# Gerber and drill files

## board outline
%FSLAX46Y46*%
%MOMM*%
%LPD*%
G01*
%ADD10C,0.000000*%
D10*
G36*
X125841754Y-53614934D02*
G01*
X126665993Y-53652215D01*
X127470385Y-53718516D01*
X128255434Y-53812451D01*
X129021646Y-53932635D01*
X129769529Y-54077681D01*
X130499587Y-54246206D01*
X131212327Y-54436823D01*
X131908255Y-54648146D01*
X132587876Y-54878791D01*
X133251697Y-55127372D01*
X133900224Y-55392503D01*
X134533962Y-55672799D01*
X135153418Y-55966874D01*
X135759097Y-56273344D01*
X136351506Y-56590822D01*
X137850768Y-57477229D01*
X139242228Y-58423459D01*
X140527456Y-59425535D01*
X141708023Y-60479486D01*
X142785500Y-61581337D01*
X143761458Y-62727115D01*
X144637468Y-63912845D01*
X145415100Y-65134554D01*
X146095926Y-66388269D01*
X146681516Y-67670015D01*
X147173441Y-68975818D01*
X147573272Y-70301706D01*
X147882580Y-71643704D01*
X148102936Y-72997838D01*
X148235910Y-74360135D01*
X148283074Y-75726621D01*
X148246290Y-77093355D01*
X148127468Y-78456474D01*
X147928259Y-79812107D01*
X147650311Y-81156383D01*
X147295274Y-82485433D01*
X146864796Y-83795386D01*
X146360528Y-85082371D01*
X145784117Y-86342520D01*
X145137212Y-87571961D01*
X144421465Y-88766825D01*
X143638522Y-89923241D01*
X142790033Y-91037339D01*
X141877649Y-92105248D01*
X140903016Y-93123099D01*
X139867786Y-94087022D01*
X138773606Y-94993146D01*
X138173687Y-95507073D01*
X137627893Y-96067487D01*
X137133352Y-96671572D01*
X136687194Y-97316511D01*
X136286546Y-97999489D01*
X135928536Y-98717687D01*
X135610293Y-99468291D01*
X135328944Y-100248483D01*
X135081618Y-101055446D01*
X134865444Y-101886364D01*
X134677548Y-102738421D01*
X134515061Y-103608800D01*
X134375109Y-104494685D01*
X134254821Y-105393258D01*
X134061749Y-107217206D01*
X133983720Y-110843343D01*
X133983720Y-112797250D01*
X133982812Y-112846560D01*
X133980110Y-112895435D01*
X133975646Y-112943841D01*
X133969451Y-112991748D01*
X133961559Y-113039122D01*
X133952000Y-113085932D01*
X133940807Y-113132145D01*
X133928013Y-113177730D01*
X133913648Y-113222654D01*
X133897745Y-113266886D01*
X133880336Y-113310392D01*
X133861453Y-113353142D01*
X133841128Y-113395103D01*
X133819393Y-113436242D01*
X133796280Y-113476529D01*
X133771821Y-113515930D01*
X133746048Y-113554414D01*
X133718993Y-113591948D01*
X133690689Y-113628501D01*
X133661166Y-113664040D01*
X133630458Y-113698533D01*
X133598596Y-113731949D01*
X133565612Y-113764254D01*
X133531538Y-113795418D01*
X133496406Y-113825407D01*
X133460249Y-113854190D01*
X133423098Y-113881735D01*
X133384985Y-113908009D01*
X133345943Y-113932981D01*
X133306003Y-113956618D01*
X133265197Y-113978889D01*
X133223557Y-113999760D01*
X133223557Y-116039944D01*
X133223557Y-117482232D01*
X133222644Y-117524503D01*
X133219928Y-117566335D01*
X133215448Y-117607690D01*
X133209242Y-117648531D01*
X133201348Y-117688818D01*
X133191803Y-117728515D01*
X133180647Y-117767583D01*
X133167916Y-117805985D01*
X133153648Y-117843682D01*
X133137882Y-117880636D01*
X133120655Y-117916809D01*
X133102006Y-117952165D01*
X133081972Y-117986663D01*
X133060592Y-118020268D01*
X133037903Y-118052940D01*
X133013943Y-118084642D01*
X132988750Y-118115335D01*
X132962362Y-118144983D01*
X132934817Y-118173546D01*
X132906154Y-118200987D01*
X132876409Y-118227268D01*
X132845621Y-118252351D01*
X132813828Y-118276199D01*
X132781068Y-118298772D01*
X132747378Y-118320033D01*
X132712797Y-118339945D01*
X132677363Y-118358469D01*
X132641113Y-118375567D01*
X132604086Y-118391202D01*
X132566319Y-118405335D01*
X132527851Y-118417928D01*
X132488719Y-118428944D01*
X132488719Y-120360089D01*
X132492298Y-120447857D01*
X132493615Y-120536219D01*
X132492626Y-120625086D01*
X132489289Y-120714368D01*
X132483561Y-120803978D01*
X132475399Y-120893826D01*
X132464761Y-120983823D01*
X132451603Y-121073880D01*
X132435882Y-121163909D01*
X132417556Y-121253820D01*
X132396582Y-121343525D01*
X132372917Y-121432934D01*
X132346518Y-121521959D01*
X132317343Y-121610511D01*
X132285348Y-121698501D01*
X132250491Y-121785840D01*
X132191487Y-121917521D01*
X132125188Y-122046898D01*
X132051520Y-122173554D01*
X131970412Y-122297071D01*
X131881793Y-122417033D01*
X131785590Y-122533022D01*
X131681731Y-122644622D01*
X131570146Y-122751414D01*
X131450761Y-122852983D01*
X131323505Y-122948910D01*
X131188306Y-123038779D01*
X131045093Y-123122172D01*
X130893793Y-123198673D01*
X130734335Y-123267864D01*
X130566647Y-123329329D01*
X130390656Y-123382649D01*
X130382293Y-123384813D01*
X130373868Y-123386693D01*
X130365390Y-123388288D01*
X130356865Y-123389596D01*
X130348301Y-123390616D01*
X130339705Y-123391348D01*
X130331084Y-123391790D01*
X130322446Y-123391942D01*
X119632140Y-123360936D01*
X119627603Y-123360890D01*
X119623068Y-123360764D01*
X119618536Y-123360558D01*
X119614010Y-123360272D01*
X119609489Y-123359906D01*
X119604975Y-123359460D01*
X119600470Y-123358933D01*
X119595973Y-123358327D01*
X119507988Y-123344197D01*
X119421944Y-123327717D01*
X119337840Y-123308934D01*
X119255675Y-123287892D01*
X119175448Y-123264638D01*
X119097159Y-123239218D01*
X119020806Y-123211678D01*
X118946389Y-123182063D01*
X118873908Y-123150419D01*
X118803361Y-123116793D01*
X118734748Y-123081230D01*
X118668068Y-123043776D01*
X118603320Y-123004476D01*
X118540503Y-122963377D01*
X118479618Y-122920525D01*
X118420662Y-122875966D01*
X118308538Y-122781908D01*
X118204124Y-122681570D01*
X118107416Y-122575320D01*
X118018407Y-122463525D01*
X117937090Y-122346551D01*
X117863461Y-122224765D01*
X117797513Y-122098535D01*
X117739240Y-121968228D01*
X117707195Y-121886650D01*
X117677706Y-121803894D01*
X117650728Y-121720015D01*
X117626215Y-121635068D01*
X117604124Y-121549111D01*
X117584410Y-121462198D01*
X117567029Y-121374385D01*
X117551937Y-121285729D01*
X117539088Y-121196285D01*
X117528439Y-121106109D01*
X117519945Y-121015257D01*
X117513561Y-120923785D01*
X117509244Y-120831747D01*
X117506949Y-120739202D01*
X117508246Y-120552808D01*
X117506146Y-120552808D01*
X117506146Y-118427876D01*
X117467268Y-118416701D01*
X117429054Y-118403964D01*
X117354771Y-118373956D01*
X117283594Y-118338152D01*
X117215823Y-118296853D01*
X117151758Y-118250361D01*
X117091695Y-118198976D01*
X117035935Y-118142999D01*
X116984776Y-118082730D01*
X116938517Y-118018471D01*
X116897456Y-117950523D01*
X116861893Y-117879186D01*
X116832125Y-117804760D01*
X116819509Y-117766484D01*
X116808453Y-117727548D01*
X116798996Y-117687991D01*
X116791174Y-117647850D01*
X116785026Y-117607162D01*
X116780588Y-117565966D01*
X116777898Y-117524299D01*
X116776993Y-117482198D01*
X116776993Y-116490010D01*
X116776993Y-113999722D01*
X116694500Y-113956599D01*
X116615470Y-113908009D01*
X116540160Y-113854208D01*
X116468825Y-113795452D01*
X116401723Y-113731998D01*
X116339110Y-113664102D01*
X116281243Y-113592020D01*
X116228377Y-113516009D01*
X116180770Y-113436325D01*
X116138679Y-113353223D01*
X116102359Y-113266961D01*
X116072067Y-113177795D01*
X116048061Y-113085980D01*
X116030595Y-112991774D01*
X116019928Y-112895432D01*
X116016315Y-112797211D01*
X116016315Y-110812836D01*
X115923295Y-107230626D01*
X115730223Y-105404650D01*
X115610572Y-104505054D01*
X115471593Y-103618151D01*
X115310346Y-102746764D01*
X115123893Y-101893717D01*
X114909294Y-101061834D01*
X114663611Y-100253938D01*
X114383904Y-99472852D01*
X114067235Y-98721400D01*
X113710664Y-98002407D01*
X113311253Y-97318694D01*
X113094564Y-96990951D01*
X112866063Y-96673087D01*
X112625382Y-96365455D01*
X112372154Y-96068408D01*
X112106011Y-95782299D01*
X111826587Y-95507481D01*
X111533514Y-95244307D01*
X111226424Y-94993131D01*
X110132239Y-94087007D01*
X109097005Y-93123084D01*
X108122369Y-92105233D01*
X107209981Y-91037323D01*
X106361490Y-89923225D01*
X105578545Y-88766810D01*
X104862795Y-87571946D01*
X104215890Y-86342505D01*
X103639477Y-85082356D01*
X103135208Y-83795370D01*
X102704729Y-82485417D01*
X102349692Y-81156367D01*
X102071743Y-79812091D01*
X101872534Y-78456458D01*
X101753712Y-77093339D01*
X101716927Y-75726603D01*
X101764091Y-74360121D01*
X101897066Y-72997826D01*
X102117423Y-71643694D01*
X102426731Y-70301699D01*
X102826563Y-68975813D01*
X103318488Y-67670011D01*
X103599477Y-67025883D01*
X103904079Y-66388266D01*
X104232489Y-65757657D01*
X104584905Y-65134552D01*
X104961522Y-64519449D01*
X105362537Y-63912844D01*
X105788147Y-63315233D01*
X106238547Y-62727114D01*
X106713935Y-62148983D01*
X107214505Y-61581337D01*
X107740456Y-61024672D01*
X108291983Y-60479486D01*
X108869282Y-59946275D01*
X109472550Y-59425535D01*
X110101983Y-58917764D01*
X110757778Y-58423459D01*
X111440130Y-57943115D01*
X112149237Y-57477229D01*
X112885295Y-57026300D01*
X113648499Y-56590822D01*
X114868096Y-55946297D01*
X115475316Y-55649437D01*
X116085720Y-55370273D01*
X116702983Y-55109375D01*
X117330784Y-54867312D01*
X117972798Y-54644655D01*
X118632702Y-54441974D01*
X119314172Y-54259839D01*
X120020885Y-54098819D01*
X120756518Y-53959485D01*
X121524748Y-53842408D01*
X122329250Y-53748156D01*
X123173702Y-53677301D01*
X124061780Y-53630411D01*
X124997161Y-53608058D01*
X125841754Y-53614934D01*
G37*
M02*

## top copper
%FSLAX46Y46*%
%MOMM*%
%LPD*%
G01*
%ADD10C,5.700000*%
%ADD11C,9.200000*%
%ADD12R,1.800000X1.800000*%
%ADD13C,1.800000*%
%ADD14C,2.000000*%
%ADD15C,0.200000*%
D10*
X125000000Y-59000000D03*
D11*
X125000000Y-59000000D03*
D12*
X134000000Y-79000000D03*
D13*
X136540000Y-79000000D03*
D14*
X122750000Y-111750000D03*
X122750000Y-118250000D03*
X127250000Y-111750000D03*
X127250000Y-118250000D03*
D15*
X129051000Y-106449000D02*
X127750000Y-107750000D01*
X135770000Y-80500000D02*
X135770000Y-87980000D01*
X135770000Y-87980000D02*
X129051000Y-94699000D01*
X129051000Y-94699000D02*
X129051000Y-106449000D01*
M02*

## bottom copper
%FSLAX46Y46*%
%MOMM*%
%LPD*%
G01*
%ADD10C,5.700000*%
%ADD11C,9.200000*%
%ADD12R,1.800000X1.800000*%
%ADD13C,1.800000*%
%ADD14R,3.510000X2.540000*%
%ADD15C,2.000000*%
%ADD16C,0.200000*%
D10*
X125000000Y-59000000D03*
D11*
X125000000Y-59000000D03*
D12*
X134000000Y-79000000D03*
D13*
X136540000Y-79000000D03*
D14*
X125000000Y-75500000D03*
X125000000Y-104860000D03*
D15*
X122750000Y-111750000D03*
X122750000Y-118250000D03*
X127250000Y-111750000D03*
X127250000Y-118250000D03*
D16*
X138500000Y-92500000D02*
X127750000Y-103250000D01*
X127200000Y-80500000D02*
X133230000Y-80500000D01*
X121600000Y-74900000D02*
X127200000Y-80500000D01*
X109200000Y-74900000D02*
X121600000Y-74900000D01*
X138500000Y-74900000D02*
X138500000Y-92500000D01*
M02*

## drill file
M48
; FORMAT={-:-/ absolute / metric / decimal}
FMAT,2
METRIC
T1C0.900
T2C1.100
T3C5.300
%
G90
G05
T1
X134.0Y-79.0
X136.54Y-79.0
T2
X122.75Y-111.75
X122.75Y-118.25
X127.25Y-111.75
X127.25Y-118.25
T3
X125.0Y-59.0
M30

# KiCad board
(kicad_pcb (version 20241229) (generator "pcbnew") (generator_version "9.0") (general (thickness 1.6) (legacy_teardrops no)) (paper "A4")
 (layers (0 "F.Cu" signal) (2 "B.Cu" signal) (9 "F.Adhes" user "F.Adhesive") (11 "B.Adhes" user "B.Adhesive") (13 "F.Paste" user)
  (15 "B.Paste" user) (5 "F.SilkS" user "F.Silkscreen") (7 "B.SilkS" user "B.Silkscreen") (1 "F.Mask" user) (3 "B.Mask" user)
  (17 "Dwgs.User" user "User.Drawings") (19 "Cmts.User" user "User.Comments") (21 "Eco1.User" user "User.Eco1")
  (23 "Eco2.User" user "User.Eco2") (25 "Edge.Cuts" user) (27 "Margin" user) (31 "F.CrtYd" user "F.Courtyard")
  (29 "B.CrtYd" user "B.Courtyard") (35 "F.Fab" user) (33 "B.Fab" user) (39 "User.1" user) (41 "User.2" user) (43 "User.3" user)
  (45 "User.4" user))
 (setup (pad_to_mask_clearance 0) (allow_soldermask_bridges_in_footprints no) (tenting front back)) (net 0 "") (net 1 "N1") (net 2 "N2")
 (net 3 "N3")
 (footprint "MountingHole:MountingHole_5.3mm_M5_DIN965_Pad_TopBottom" (layer "F.Cu") (at 125 59)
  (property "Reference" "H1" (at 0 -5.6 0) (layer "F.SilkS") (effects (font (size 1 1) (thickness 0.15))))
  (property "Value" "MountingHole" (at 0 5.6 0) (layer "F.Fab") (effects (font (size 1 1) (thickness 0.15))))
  (pad "1" thru_hole circle (at 0 0) (size 5.7 5.7) (drill 5.3) (layers "*.Cu" "*.Mask") (remove_unused_layers no))
  (pad "1" connect circle (at 0 0) (size 9.2 9.2) (layers "F.Cu" "F.Mask"))
  (pad "1" connect circle (at 0 0) (size 9.2 9.2) (layers "B.Cu" "B.Mask")))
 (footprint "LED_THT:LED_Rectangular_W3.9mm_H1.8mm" (layer "F.Cu") (at 134 79)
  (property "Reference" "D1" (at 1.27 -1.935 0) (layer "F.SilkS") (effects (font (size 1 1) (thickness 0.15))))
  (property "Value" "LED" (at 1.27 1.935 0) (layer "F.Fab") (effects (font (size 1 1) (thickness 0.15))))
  (pad "1" thru_hole rect (at 0 0) (size 1.8 1.8) (drill 0.9) (layers "*.Cu" "*.Mask") (remove_unused_layers no) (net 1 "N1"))
  (pad "2" thru_hole circle (at 2.54 0) (size 1.8 1.8) (drill 0.9) (layers "*.Cu" "*.Mask") (remove_unused_layers no) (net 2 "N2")))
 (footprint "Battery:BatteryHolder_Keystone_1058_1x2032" (layer "B.Cu") (at 125 90.18 -90)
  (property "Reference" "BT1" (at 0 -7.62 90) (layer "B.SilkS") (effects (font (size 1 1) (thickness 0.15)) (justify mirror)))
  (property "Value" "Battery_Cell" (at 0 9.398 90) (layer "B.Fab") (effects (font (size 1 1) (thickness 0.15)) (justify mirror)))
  (pad "1" smd rect (at -14.68 0 270) (size 2.54 3.51) (layers "B.Cu" "B.Mask" "B.Paste") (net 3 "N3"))
  (pad "2" smd rect (at 14.68 0 270) (size 2.54 3.51) (layers "B.Cu" "B.Mask" "B.Paste") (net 1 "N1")))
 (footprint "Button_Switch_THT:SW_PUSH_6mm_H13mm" (layer "B.Cu") (at 122.75 111.75 -90)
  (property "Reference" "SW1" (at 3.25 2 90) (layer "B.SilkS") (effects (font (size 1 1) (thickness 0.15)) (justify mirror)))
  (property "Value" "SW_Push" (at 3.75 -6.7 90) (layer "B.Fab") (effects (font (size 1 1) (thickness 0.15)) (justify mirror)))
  (pad "1" thru_hole circle (at 0 0 180) (size 2 2) (drill 1.1) (layers "*.Cu" "*.Mask") (remove_unused_layers no) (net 3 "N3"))
  (pad "1" thru_hole circle (at 6.5 0 180) (size 2 2) (drill 1.1) (layers "*.Cu" "*.Mask") (remove_unused_layers no) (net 3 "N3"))
  (pad "2" thru_hole circle (at 0 -4.5 180) (size 2 2) (drill 1.1) (layers "*.Cu" "*.Mask") (remove_unused_layers no) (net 2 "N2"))
  (pad "2" thru_hole circle (at 6.5 -4.5 180) (size 2 2) (drill 1.1) (layers "*.Cu" "*.Mask") (remove_unused_layers no) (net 2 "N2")))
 (gr_poly
  (pts (xy 125.841754 53.614934) (xy 126.665993 53.652215) (xy 127.470385 53.718516) (xy 128.255434 53.812451) (xy 129.021646 53.932635)
   (xy 129.769529 54.077681) (xy 130.499587 54.246206) (xy 131.212327 54.436823) (xy 131.908255 54.648146) (xy 132.587876 54.878791)
   (xy 133.251697 55.127372) (xy 133.900224 55.392503) (xy 134.533962 55.672799) (xy 135.153418 55.966874) (xy 135.759097 56.273344)
   (xy 136.351506 56.590822) (xy 137.850768 57.477229) (xy 139.242228 58.423459) (xy 140.527456 59.425535) (xy 141.708023 60.479486)
   (xy 142.7855 61.581337) (xy 143.761458 62.727115) (xy 144.637468 63.912845) (xy 145.4151 65.134554) (xy 146.095926 66.388269)
   (xy 146.681516 67.670015) (xy 147.173441 68.975818) (xy 147.573272 70.301706) (xy 147.88258 71.643704) (xy 148.102936 72.997838)
   (xy 148.23591 74.360135) (xy 148.283074 75.726621) (xy 148.24629 77.093355) (xy 148.127468 78.456474) (xy 147.928259 79.812107)
   (xy 147.650311 81.156383) (xy 147.295274 82.485433) (xy 146.864796 83.795386) (xy 146.360528 85.082371) (xy 145.784117 86.34252)
   (xy 145.137212 87.571961) (xy 144.421465 88.766825) (xy 143.638522 89.923241) (xy 142.790033 91.037339) (xy 141.877649 92.105248)
   (xy 140.903016 93.123099) (xy 139.867786 94.087022) (xy 138.773606 94.993146) (xy 138.173687 95.507073) (xy 137.627893 96.067487)
   (xy 137.133352 96.671572) (xy 136.687194 97.316511) (xy 136.286546 97.999489) (xy 135.928536 98.717687) (xy 135.610293 99.468291)
   (xy 135.328944 100.248483) (xy 135.081618 101.055446) (xy 134.865444 101.886364) (xy 134.677548 102.738421) (xy 134.515061 103.6088)
   (xy 134.375109 104.494685) (xy 134.254821 105.393258) (xy 134.061749 107.217206) (xy 133.98372 110.843343) (xy 133.98372 112.79725)
   (xy 133.982812 112.84656) (xy 133.98011 112.895435) (xy 133.975646 112.943841) (xy 133.969451 112.991748) (xy 133.961559 113.039122)
   (xy 133.952 113.085932) (xy 133.940807 113.132145) (xy 133.928013 113.17773) (xy 133.913648 113.222654) (xy 133.897745 113.266886)
   (xy 133.880336 113.310392) (xy 133.861453 113.353142) (xy 133.841128 113.395103) (xy 133.819393 113.436242) (xy 133.79628 113.476529)
   (xy 133.771821 113.51593) (xy 133.746048 113.554414) (xy 133.718993 113.591948) (xy 133.690689 113.628501) (xy 133.661166 113.66404)
   (xy 133.630458 113.698533) (xy 133.598596 113.731949) (xy 133.565612 113.764254) (xy 133.531538 113.795418) (xy 133.496406 113.825407)
   (xy 133.460249 113.85419) (xy 133.423098 113.881735) (xy 133.384985 113.908009) (xy 133.345943 113.932981) (xy 133.306003 113.956618)
   (xy 133.265197 113.978889) (xy 133.223557 113.99976) (xy 133.223557 116.039944) (xy 133.223557 117.482232) (xy 133.222644 117.524503)
   (xy 133.219928 117.566335) (xy 133.215448 117.60769) (xy 133.209242 117.648531) (xy 133.201348 117.688818) (xy 133.191803 117.728515)
   (xy 133.180647 117.767583) (xy 133.167916 117.805985) (xy 133.153648 117.843682) (xy 133.137882 117.880636) (xy 133.120655 117.916809)
   (xy 133.102006 117.952165) (xy 133.081972 117.986663) (xy 133.060592 118.020268) (xy 133.037903 118.05294) (xy 133.013943 118.084642)
   (xy 132.98875 118.115335) (xy 132.962362 118.144983) (xy 132.934817 118.173546) (xy 132.906154 118.200987) (xy 132.876409 118.227268)
   (xy 132.845621 118.252351) (xy 132.813828 118.276199) (xy 132.781068 118.298772) (xy 132.747378 118.320033) (xy 132.712797 118.339945)
   (xy 132.677363 118.358469) (xy 132.641113 118.375567) (xy 132.604086 118.391202) (xy 132.566319 118.405335) (xy 132.527851 118.417928)
   (xy 132.488719 118.428944) (xy 132.488719 120.360089) (xy 132.492298 120.447857) (xy 132.493615 120.536219) (xy 132.492626 120.625086)
   (xy 132.489289 120.714368) (xy 132.483561 120.803978) (xy 132.475399 120.893826) (xy 132.464761 120.983823) (xy 132.451603 121.07388)
   (xy 132.435882 121.163909) (xy 132.417556 121.25382) (xy 132.396582 121.343525) (xy 132.372917 121.432934) (xy 132.346518 121.521959)
   (xy 132.317343 121.610511) (xy 132.285348 121.698501) (xy 132.250491 121.78584) (xy 132.191487 121.917521) (xy 132.125188 122.046898)
   (xy 132.05152 122.173554) (xy 131.970412 122.297071) (xy 131.881793 122.417033) (xy 131.78559 122.533022) (xy 131.681731 122.644622)
   (xy 131.570146 122.751414) (xy 131.450761 122.852983) (xy 131.323505 122.94891) (xy 131.188306 123.038779) (xy 131.045093 123.122172)
   (xy 130.893793 123.198673) (xy 130.734335 123.267864) (xy 130.566647 123.329329) (xy 130.390656 123.382649) (xy 130.382293 123.384813)
   (xy 130.373868 123.386693) (xy 130.36539 123.388288) (xy 130.356865 123.389596) (xy 130.348301 123.390616) (xy 130.339705 123.391348)
   (xy 130.331084 123.39179) (xy 130.322446 123.391942) (xy 119.63214 123.360936) (xy 119.627603 123.36089) (xy 119.623068 123.360764)
   (xy 119.618536 123.360558) (xy 119.61401 123.360272) (xy 119.609489 123.359906) (xy 119.604975 123.35946) (xy 119.60047 123.358933)
   (xy 119.595973 123.358327) (xy 119.507988 123.344197) (xy 119.421944 123.327717) (xy 119.33784 123.308934) (xy 119.255675 123.287892)
   (xy 119.175448 123.264638) (xy 119.097159 123.239218) (xy 119.020806 123.211678) (xy 118.946389 123.182063) (xy 118.873908 123.150419)
   (xy 118.803361 123.116793) (xy 118.734748 123.08123) (xy 118.668068 123.043776) (xy 118.60332 123.004476) (xy 118.540503 122.963377)
   (xy 118.479618 122.920525) (xy 118.420662 122.875966) (xy 118.308538 122.781908) (xy 118.204124 122.68157) (xy 118.107416 122.57532)
   (xy 118.018407 122.463525) (xy 117.93709 122.346551) (xy 117.863461 122.224765) (xy 117.797513 122.098535) (xy 117.73924 121.968228)
   (xy 117.707195 121.88665) (xy 117.677706 121.803894) (xy 117.650728 121.720015) (xy 117.626215 121.635068) (xy 117.604124 121.549111)
   (xy 117.58441 121.462198) (xy 117.567029 121.374385) (xy 117.551937 121.285729) (xy 117.539088 121.196285) (xy 117.528439 121.106109)
   (xy 117.519945 121.015257) (xy 117.513561 120.923785) (xy 117.509244 120.831747) (xy 117.506949 120.739202) (xy 117.508246 120.552808)
   (xy 117.506146 120.552808) (xy 117.506146 118.427876) (xy 117.467268 118.416701) (xy 117.429054 118.403964) (xy 117.354771 118.373956)
   (xy 117.283594 118.338152) (xy 117.215823 118.296853) (xy 117.151758 118.250361) (xy 117.091695 118.198976) (xy 117.035935 118.142999)
   (xy 116.984776 118.08273) (xy 116.938517 118.018471) (xy 116.897456 117.950523) (xy 116.861893 117.879186) (xy 116.832125 117.80476)
   (xy 116.819509 117.766484) (xy 116.808453 117.727548) (xy 116.798996 117.687991) (xy 116.791174 117.64785) (xy 116.785026 117.607162)
   (xy 116.780588 117.565966) (xy 116.777898 117.524299) (xy 116.776993 117.482198) (xy 116.776993 116.49001) (xy 116.776993 113.999722)
   (xy 116.6945 113.956599) (xy 116.61547 113.908009) (xy 116.54016 113.854208) (xy 116.468825 113.795452) (xy 116.401723 113.731998)
   (xy 116.33911 113.664102) (xy 116.281243 113.59202) (xy 116.228377 113.516009) (xy 116.18077 113.436325) (xy 116.138679 113.353223)
   (xy 116.102359 113.266961) (xy 116.072067 113.177795) (xy 116.048061 113.08598) (xy 116.030595 112.991774) (xy 116.019928 112.895432)
   (xy 116.016315 112.797211) (xy 116.016315 110.812836) (xy 115.923295 107.230626) (xy 115.730223 105.40465) (xy 115.610572 104.505054)
   (xy 115.471593 103.618151) (xy 115.310346 102.746764) (xy 115.123893 101.893717) (xy 114.909294 101.061834) (xy 114.663611 100.253938)
   (xy 114.383904 99.472852) (xy 114.067235 98.7214) (xy 113.710664 98.002407) (xy 113.311253 97.318694) (xy 113.094564 96.990951)
   (xy 112.866063 96.673087) (xy 112.625382 96.365455) (xy 112.372154 96.068408) (xy 112.106011 95.782299) (xy 111.826587 95.507481)
   (xy 111.533514 95.244307) (xy 111.226424 94.993131) (xy 110.132239 94.087007) (xy 109.097005 93.123084) (xy 108.122369 92.105233)
   (xy 107.209981 91.037323) (xy 106.36149 89.923225) (xy 105.578545 88.76681) (xy 104.862795 87.571946) (xy 104.21589 86.342505)
   (xy 103.639477 85.082356) (xy 103.135208 83.79537) (xy 102.704729 82.485417) (xy 102.349692 81.156367) (xy 102.071743 79.812091)
   (xy 101.872534 78.456458) (xy 101.753712 77.093339) (xy 101.716927 75.726603) (xy 101.764091 74.360121) (xy 101.897066 72.997826)
   (xy 102.117423 71.643694) (xy 102.426731 70.301699) (xy 102.826563 68.975813) (xy 103.318488 67.670011) (xy 103.599477 67.025883)
   (xy 103.904079 66.388266) (xy 104.232489 65.757657) (xy 104.584905 65.134552) (xy 104.961522 64.519449) (xy 105.362537 63.912844)
   (xy 105.788147 63.315233) (xy 106.238547 62.727114) (xy 106.713935 62.148983) (xy 107.214505 61.581337) (xy 107.740456 61.024672)
   (xy 108.291983 60.479486) (xy 108.869282 59.946275) (xy 109.47255 59.425535) (xy 110.101983 58.917764) (xy 110.757778 58.423459)
   (xy 111.44013 57.943115) (xy 112.149237 57.477229) (xy 112.885295 57.0263) (xy 113.648499 56.590822) (xy 114.868096 55.946297)
   (xy 115.475316 55.649437) (xy 116.08572 55.370273) (xy 116.702983 55.109375) (xy 117.330784 54.867312) (xy 117.972798 54.644655)
   (xy 118.632702 54.441974) (xy 119.314172 54.259839) (xy 120.020885 54.098819) (xy 120.756518 53.959485) (xy 121.524748 53.842408)
   (xy 122.32925 53.748156) (xy 123.173702 53.677301) (xy 124.06178 53.630411) (xy 124.997161 53.608058))
  (stroke (width 0) (type solid)) (fill yes) (layer "Edge.Cuts"))
 (segment (start 138.5 92.5) (end 127.75 103.25) (width 0.2) (layer "B.Cu") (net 3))
 (segment (start 127.2 80.5) (end 133.23 80.5) (width 0.2) (layer "B.Cu") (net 3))
 (segment (start 121.6 74.9) (end 127.2 80.5) (width 0.2) (layer "B.Cu") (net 3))
 (segment (start 109.2 74.9) (end 121.6 74.9) (width 0.2) (layer "B.Cu") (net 3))
 (segment (start 138.5 74.9) (end 138.5 92.5) (width 0.2) (layer "B.Cu") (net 3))
 (segment (start 129.051 106.449) (end 127.75 107.75) (width 0.2) (layer "F.Cu") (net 2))
 (segment (start 135.77 80.5) (end 135.77 87.98) (width 0.2) (layer "F.Cu") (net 2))
 (segment (start 135.77 87.98) (end 129.051 94.699) (width 0.2) (layer "F.Cu") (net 2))
 (segment (start 129.051 94.699) (end 129.051 106.449) (width 0.2) (layer "F.Cu") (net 2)))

